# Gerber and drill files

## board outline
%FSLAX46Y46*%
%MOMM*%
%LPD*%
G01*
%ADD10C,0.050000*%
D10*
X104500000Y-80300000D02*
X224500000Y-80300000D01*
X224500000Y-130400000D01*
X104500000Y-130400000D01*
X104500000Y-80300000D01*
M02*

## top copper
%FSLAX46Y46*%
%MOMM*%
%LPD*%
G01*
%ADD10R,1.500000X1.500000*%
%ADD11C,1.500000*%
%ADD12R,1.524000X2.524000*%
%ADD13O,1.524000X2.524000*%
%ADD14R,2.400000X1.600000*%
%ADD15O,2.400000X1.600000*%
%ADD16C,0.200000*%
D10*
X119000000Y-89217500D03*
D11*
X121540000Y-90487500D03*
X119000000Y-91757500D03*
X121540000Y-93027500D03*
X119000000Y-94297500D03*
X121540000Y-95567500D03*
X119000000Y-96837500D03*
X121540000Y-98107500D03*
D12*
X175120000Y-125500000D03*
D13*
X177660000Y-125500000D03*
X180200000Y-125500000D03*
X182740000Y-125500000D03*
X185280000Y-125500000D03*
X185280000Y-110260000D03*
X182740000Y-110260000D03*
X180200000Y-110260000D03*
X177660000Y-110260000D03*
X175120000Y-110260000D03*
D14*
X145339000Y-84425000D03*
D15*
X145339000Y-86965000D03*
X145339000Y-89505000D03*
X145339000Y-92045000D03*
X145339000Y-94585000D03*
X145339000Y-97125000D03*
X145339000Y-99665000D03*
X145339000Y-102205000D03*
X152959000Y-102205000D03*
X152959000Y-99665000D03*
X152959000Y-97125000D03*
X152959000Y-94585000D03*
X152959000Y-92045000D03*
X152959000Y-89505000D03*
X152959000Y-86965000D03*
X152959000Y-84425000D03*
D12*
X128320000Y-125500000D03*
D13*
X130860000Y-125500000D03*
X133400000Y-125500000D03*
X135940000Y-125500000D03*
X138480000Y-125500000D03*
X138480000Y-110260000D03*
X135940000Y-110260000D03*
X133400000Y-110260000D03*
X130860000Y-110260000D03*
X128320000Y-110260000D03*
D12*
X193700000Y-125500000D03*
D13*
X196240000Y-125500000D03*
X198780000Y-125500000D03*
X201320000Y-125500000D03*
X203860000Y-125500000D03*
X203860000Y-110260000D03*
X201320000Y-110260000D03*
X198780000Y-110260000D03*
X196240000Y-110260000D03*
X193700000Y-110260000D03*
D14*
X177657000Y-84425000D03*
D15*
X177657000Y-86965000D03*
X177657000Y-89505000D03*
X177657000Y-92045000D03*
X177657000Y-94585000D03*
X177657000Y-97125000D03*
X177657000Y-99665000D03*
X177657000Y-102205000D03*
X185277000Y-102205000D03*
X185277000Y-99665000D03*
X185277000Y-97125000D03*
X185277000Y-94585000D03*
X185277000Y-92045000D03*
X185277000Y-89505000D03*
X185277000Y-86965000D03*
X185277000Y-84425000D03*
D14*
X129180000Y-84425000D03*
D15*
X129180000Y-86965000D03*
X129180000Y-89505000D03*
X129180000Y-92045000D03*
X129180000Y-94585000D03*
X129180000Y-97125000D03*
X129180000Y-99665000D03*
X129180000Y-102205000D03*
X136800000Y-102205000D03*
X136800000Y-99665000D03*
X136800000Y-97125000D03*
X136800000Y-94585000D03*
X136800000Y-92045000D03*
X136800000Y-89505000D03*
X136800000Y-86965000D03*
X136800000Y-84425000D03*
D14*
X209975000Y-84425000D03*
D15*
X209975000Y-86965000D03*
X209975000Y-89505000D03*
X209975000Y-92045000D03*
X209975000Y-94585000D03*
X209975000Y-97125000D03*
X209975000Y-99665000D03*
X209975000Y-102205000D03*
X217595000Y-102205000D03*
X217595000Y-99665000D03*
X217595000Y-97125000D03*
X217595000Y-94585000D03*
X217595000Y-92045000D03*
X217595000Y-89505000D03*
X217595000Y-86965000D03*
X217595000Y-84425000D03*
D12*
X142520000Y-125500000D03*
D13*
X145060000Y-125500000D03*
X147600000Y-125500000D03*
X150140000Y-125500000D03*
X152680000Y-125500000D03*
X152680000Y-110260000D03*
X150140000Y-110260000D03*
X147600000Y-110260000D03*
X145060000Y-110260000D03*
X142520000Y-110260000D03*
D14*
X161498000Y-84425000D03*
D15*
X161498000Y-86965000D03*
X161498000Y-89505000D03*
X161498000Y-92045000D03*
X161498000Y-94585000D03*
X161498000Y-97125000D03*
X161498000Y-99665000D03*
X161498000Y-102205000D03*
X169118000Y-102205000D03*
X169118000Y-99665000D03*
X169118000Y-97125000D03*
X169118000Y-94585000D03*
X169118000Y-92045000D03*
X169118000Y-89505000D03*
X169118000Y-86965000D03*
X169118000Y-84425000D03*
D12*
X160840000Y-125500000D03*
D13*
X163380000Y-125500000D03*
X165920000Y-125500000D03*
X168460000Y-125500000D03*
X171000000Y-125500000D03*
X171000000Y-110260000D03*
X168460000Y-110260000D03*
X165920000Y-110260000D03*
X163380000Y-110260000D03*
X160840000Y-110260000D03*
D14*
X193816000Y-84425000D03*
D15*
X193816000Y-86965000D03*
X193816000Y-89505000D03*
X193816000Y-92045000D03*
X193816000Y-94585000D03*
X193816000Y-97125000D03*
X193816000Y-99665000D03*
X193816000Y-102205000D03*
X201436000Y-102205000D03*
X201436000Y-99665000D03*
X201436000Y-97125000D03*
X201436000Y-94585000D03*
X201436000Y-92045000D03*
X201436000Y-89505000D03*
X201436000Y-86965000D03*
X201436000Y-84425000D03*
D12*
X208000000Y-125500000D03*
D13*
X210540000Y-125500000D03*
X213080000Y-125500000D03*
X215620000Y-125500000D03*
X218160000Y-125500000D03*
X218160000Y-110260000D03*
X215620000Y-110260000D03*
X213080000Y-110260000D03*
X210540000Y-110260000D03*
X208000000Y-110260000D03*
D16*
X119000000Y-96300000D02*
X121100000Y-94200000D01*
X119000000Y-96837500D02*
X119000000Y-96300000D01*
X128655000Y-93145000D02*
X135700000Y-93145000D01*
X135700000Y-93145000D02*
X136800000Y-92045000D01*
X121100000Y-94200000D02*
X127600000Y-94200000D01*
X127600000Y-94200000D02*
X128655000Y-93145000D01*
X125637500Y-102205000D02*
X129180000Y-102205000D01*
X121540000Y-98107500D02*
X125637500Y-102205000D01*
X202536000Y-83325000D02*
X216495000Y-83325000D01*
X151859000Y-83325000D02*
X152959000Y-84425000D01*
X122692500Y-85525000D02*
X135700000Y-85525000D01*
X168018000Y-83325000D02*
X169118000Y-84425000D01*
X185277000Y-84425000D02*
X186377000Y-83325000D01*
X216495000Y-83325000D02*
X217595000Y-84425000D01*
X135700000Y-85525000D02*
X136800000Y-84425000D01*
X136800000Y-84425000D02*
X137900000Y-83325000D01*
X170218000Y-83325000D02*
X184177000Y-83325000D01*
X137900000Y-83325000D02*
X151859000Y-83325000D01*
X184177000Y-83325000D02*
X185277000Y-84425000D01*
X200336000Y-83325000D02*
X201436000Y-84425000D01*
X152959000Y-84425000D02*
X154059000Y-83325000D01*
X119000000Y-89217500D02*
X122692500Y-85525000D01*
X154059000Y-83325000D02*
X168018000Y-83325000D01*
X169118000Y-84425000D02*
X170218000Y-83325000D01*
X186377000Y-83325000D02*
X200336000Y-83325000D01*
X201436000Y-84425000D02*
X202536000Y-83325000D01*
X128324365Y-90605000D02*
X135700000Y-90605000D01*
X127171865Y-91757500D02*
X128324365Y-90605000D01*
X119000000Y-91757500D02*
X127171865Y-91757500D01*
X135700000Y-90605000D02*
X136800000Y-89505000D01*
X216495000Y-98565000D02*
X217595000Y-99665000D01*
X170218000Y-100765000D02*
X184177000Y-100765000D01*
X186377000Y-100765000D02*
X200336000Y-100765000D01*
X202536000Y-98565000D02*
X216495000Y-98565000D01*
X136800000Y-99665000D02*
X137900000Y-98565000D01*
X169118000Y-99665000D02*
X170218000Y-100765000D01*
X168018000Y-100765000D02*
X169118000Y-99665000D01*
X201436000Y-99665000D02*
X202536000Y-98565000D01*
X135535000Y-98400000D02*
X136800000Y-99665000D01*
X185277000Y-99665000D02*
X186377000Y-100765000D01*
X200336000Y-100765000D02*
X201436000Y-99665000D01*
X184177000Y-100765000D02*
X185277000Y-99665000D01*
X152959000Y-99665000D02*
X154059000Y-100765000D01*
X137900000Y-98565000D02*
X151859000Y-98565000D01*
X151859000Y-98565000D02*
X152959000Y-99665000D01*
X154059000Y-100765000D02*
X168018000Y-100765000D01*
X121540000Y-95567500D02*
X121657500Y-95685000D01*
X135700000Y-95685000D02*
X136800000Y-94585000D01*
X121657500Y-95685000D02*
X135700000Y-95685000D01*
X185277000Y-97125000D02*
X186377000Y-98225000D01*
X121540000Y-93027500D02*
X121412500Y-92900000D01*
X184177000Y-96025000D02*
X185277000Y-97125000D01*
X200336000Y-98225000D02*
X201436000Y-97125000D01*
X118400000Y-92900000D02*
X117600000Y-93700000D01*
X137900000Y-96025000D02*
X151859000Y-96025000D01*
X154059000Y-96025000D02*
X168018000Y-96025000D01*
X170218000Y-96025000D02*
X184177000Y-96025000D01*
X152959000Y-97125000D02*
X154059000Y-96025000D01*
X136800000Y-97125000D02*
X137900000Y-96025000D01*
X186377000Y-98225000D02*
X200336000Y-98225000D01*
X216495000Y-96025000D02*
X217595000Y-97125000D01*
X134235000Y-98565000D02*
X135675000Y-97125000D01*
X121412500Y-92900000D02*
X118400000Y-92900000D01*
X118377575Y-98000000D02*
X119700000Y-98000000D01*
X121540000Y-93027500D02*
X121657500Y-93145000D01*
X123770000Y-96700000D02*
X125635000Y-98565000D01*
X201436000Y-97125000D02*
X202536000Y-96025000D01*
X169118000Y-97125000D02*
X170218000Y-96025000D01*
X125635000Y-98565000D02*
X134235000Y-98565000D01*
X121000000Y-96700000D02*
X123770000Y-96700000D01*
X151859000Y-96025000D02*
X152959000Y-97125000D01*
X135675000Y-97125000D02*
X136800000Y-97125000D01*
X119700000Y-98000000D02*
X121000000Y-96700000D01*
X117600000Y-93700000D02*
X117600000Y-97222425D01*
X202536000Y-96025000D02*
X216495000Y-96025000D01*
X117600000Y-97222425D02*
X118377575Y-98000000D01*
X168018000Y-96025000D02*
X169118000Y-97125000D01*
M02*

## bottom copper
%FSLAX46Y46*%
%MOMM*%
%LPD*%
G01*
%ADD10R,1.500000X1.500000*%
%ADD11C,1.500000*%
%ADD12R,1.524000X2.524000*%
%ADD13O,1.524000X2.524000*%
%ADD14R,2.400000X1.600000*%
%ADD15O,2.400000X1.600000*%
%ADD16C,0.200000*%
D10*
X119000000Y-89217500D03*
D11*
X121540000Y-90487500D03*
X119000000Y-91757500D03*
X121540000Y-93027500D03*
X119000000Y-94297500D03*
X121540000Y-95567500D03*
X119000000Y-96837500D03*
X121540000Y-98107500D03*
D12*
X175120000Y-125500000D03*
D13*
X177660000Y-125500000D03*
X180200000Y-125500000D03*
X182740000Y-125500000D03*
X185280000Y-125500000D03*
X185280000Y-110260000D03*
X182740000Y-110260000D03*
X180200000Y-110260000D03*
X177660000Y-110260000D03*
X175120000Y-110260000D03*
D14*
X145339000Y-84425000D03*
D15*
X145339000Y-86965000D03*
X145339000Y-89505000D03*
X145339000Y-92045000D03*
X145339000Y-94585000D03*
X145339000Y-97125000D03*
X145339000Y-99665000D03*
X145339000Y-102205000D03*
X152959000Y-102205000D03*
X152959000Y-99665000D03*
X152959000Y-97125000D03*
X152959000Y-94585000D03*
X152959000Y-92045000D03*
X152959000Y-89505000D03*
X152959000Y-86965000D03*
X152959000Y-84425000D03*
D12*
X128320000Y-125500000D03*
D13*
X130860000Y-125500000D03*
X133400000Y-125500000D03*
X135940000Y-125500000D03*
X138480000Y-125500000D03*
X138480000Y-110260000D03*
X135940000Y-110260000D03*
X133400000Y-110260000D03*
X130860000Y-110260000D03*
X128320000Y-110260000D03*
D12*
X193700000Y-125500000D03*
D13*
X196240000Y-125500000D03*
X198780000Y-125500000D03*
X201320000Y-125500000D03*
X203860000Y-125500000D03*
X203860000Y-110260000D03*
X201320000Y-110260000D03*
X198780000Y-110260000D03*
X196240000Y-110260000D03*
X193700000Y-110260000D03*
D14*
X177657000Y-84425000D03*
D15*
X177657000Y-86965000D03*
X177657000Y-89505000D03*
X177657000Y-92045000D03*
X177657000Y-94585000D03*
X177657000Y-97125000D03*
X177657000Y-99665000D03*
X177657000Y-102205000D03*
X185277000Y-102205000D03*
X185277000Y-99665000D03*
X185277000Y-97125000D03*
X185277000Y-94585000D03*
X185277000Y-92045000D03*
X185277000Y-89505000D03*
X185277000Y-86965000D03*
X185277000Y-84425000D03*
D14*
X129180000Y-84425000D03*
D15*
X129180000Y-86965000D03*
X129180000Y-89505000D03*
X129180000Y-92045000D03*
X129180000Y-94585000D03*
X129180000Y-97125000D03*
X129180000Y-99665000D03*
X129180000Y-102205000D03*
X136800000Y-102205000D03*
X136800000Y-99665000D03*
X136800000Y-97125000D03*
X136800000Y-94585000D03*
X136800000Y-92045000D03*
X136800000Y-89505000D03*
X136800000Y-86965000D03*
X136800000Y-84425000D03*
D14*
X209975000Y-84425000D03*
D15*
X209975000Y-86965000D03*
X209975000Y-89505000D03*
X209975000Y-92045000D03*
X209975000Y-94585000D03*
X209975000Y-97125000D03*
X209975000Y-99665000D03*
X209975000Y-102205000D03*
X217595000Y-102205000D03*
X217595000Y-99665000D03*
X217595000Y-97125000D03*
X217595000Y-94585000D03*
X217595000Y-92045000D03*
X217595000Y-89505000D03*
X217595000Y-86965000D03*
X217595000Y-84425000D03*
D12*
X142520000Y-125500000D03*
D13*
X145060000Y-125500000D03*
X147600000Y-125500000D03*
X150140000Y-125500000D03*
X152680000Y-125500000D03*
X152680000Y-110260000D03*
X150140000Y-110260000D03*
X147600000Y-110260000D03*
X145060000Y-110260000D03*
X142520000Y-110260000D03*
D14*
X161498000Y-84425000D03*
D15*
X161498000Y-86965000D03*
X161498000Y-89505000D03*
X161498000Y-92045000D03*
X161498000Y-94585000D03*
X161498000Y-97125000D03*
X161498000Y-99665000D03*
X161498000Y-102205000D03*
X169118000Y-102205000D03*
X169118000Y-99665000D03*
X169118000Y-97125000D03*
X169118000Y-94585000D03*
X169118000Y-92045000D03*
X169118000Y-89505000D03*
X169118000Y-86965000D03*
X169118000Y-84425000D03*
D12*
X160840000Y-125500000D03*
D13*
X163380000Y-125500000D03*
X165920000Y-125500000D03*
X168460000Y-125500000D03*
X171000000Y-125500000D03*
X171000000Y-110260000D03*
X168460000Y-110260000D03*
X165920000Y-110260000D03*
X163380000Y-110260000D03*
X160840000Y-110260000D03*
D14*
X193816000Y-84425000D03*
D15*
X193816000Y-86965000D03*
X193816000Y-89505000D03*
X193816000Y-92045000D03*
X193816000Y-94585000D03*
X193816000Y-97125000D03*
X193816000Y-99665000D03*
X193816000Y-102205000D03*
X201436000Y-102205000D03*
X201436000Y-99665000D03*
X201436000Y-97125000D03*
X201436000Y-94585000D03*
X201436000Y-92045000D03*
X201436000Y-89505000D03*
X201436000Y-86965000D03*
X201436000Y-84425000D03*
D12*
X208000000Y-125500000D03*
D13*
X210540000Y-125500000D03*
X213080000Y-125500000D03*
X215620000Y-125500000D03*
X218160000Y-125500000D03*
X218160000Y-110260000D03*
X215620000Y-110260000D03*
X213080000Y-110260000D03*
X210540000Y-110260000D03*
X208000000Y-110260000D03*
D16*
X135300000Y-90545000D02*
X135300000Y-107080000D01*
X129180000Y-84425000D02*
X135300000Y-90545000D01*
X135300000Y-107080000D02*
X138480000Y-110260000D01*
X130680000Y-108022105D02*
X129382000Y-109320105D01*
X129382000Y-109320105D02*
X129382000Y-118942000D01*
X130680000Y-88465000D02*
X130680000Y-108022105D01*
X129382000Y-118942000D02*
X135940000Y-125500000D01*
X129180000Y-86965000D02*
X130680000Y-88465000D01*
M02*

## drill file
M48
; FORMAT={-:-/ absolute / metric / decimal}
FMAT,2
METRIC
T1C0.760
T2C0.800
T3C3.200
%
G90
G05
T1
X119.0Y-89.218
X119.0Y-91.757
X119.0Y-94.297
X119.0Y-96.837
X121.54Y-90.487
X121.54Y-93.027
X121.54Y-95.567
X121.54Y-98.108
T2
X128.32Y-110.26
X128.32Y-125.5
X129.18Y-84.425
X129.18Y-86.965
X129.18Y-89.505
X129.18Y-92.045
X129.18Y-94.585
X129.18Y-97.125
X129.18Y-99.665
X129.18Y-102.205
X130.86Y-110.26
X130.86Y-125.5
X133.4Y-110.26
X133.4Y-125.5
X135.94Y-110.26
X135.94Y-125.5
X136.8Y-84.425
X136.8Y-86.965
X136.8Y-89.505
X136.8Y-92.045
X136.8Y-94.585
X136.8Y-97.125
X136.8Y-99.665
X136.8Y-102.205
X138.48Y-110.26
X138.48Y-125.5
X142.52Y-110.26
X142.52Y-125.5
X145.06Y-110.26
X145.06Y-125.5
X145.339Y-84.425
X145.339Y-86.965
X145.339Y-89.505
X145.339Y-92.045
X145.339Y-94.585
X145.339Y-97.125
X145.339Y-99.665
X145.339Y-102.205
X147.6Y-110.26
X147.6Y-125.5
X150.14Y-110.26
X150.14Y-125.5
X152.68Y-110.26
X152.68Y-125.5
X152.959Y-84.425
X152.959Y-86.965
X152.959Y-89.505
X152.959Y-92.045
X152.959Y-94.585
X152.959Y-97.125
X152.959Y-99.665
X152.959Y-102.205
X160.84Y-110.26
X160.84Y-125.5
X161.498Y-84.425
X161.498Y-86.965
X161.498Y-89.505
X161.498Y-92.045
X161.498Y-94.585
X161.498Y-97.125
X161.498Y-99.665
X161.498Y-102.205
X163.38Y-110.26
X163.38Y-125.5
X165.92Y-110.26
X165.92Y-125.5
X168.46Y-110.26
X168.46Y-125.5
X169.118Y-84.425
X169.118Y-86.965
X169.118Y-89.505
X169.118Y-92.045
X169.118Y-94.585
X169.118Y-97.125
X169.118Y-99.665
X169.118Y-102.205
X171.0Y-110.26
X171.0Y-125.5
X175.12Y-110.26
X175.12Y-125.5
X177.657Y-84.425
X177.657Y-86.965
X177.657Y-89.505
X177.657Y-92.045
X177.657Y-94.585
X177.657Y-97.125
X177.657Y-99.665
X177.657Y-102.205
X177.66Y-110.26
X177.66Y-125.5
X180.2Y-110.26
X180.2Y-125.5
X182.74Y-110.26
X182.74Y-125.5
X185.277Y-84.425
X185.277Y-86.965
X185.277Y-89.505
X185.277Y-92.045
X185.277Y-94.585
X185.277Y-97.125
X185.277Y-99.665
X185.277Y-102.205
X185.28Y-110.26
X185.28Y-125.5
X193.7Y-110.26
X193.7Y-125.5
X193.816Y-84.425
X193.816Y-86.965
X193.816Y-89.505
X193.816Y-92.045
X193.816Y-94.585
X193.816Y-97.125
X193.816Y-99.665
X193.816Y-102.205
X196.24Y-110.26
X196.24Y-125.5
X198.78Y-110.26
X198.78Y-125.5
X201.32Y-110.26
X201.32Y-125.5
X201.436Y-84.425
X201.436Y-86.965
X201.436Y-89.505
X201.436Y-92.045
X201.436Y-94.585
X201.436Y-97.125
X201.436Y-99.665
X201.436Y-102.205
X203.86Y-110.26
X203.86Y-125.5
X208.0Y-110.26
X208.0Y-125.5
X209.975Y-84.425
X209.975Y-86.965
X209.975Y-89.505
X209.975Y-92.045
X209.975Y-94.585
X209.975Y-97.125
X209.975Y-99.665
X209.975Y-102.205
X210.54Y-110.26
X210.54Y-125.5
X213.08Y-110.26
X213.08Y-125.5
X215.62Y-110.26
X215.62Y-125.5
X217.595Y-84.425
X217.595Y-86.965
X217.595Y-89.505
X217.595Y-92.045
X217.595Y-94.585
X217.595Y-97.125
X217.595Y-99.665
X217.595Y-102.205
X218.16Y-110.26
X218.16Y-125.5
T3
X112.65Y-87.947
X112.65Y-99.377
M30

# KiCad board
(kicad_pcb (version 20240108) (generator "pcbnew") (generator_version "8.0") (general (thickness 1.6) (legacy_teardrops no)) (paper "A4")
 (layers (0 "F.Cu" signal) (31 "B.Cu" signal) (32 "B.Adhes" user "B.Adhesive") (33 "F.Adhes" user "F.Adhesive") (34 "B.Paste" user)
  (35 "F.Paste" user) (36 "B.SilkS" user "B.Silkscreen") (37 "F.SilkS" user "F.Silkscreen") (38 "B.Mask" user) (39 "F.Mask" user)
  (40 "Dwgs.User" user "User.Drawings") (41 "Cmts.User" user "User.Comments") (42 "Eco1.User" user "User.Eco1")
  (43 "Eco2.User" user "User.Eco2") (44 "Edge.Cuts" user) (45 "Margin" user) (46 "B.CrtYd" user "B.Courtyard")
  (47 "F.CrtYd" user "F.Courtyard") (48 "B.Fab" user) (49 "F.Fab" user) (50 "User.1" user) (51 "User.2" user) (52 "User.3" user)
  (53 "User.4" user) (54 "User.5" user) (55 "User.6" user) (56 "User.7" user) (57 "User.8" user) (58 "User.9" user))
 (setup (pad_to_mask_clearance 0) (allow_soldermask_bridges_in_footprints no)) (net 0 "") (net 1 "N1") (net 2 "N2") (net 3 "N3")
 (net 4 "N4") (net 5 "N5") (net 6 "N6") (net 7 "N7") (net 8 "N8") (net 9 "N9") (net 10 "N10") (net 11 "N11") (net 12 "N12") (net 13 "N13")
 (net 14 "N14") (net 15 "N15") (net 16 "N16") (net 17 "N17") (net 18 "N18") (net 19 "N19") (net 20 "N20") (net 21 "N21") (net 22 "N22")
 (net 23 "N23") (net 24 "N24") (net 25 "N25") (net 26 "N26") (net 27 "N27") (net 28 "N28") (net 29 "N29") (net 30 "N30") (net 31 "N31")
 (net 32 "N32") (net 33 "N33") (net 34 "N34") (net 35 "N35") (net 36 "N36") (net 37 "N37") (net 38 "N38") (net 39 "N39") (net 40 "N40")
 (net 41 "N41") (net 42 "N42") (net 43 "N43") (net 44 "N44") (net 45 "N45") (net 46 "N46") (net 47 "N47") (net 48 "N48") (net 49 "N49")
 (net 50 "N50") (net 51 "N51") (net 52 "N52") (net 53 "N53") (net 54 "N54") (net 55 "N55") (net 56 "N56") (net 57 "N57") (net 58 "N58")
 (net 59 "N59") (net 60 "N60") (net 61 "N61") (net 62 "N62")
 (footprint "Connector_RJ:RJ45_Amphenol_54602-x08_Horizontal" (layer "F.Cu") (at 119 89.2175 -90)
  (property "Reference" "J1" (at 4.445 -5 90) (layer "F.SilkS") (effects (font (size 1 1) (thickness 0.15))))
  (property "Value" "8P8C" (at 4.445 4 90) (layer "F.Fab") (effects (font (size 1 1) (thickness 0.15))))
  (pad "" np_thru_hole circle (at -1.27 6.35 270) (size 3.2 3.2) (drill 3.2) (layers "*.Cu" "*.Mask"))
  (pad "" np_thru_hole circle (at 10.16 6.35 270) (size 3.2 3.2) (drill 3.2) (layers "*.Cu" "*.Mask"))
  (pad "1" thru_hole rect (at 0 0 270) (size 1.5 1.5) (drill 0.76) (layers "*.Cu" "*.Mask") (remove_unused_layers no) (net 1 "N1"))
  (pad "2" thru_hole circle (at 1.27 -2.54 270) (size 1.5 1.5) (drill 0.76) (layers "*.Cu" "*.Mask") (remove_unused_layers no) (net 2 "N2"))
  (pad "3" thru_hole circle (at 2.54 0 270) (size 1.5 1.5) (drill 0.76) (layers "*.Cu" "*.Mask") (remove_unused_layers no) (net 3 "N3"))
  (pad "4" thru_hole circle (at 3.81 -2.54 270) (size 1.5 1.5) (drill 0.76) (layers "*.Cu" "*.Mask") (remove_unused_layers no) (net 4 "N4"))
  (pad "5" thru_hole circle (at 5.08 0 270) (size 1.5 1.5) (drill 0.76) (layers "*.Cu" "*.Mask") (remove_unused_layers no) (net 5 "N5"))
  (pad "6" thru_hole circle (at 6.35 -2.54 270) (size 1.5 1.5) (drill 0.76) (layers "*.Cu" "*.Mask") (remove_unused_layers no) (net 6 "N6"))
  (pad "7" thru_hole circle (at 7.62 0 270) (size 1.5 1.5) (drill 0.76) (layers "*.Cu" "*.Mask") (remove_unused_layers no) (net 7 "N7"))
  (pad "8" thru_hole circle (at 8.89 -2.54 270) (size 1.5 1.5) (drill 0.76) (layers "*.Cu" "*.Mask") (remove_unused_layers no) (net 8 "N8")))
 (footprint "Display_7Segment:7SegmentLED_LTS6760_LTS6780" (layer "F.Cu") (at 175.12 125.5 90)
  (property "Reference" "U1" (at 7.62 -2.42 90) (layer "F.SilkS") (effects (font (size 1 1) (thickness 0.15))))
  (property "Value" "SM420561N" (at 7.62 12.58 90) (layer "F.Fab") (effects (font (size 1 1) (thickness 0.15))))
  (pad "1" thru_hole rect (at 0 0) (size 1.524 2.524) (drill 0.8) (layers "*.Cu" "*.Mask") (remove_unused_layers no) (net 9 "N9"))
  (pad "2" thru_hole oval (at 0 2.54) (size 1.524 2.524) (drill 0.8) (layers "*.Cu" "*.Mask") (remove_unused_layers no) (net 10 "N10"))
  (pad "3" thru_hole oval (at 0 5.08) (size 1.524 2.524) (drill 0.8) (layers "*.Cu" "*.Mask") (remove_unused_layers no) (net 8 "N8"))
  (pad "4" thru_hole oval (at 0 7.62) (size 1.524 2.524) (drill 0.8) (layers "*.Cu" "*.Mask") (remove_unused_layers no) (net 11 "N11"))
  (pad "5" thru_hole oval (at 0 10.16) (size 1.524 2.524) (drill 0.8) (layers "*.Cu" "*.Mask") (remove_unused_layers no) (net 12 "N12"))
  (pad "6" thru_hole oval (at 15.24 10.16) (size 1.524 2.524) (drill 0.8) (layers "*.Cu" "*.Mask") (remove_unused_layers no) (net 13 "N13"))
  (pad "7" thru_hole oval (at 15.24 7.62) (size 1.524 2.524) (drill 0.8) (layers "*.Cu" "*.Mask") (remove_unused_layers no) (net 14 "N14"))
  (pad "8" thru_hole oval (at 15.24 5.08) (size 1.524 2.524) (drill 0.8) (layers "*.Cu" "*.Mask") (remove_unused_layers no) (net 8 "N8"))
  (pad "9" thru_hole oval (at 15.24 2.54) (size 1.524 2.524) (drill 0.8) (layers "*.Cu" "*.Mask") (remove_unused_layers no) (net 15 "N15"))
  (pad "10" thru_hole oval (at 15.24 0) (size 1.524 2.524) (drill 0.8) (layers "*.Cu" "*.Mask") (remove_unused_layers no) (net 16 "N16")))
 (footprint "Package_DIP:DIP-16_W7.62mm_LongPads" (layer "F.Cu") (at 145.339 84.425)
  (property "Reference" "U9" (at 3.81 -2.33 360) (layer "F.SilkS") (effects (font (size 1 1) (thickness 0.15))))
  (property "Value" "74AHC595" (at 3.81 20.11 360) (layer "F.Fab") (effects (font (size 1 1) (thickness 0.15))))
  (pad "1" thru_hole rect (at 0 0) (size 2.4 1.6) (drill 0.8) (layers "*.Cu" "*.Mask") (remove_unused_layers no) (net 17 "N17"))
  (pad "2" thru_hole oval (at 0 2.54) (size 2.4 1.6) (drill 0.8) (layers "*.Cu" "*.Mask") (remove_unused_layers no) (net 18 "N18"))
  (pad "3" thru_hole oval (at 0 5.08) (size 2.4 1.6) (drill 0.8) (layers "*.Cu" "*.Mask") (remove_unused_layers no) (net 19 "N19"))
  (pad "4" thru_hole oval (at 0 7.62) (size 2.4 1.6) (drill 0.8) (layers "*.Cu" "*.Mask") (remove_unused_layers no) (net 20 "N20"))
  (pad "5" thru_hole oval (at 0 10.16) (size 2.4 1.6) (drill 0.8) (layers "*.Cu" "*.Mask") (remove_unused_layers no) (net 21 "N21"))
  (pad "6" thru_hole oval (at 0 12.7) (size 2.4 1.6) (drill 0.8) (layers "*.Cu" "*.Mask") (remove_unused_layers no) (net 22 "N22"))
  (pad "7" thru_hole oval (at 0 15.24) (size 2.4 1.6) (drill 0.8) (layers "*.Cu" "*.Mask") (remove_unused_layers no) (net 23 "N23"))
  (pad "8" thru_hole oval (at 0 17.78) (size 2.4 1.6) (drill 0.8) (layers "*.Cu" "*.Mask") (remove_unused_layers no) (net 8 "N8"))
  (pad "9" thru_hole oval (at 7.62 17.78) (size 2.4 1.6) (drill 0.8) (layers "*.Cu" "*.Mask") (remove_unused_layers no) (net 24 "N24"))
  (pad "10" thru_hole oval (at 7.62 15.24) (size 2.4 1.6) (drill 0.8) (layers "*.Cu" "*.Mask") (remove_unused_layers no) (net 5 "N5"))
  (pad "11" thru_hole oval (at 7.62 12.7) (size 2.4 1.6) (drill 0.8) (layers "*.Cu" "*.Mask") (remove_unused_layers no) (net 4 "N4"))
  (pad "12" thru_hole oval (at 7.62 10.16) (size 2.4 1.6) (drill 0.8) (layers "*.Cu" "*.Mask") (remove_unused_layers no) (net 6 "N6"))
  (pad "13" thru_hole oval (at 7.62 7.62) (size 2.4 1.6) (drill 0.8) (layers "*.Cu" "*.Mask") (remove_unused_layers no) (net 7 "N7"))
  (pad "14" thru_hole oval (at 7.62 5.08) (size 2.4 1.6) (drill 0.8) (layers "*.Cu" "*.Mask") (remove_unused_layers no) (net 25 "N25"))
  (pad "15" thru_hole oval (at 7.62 2.54) (size 2.4 1.6) (drill 0.8) (layers "*.Cu" "*.Mask") (remove_unused_layers no) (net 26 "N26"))
  (pad "16" thru_hole oval (at 7.62 0) (size 2.4 1.6) (drill 0.8) (layers "*.Cu" "*.Mask") (remove_unused_layers no) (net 1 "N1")))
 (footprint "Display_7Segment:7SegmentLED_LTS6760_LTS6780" (layer "F.Cu") (at 128.32 125.5 90)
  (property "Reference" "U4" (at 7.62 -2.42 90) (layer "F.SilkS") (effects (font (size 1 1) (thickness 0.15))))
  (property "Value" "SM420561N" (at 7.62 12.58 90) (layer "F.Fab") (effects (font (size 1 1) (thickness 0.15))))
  (pad "1" thru_hole rect (at 0 0) (size 1.524 2.524) (drill 0.8) (layers "*.Cu" "*.Mask") (remove_unused_layers no) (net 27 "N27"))
  (pad "2" thru_hole oval (at 0 2.54) (size 1.524 2.524) (drill 0.8) (layers "*.Cu" "*.Mask") (remove_unused_layers no) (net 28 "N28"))
  (pad "3" thru_hole oval (at 0 5.08) (size 1.524 2.524) (drill 0.8) (layers "*.Cu" "*.Mask") (remove_unused_layers no) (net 8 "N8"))
  (pad "4" thru_hole oval (at 0 7.62) (size 1.524 2.524) (drill 0.8) (layers "*.Cu" "*.Mask") (remove_unused_layers no) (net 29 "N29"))
  (pad "5" thru_hole oval (at 0 10.16) (size 1.524 2.524) (drill 0.8) (layers "*.Cu" "*.Mask") (remove_unused_layers no) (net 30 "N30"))
  (pad "6" thru_hole oval (at 15.24 10.16) (size 1.524 2.524) (drill 0.8) (layers "*.Cu" "*.Mask") (remove_unused_layers no) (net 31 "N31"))
  (pad "7" thru_hole oval (at 15.24 7.62) (size 1.524 2.524) (drill 0.8) (layers "*.Cu" "*.Mask") (remove_unused_layers no) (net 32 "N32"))
  (pad "8" thru_hole oval (at 15.24 5.08) (size 1.524 2.524) (drill 0.8) (layers "*.Cu" "*.Mask") (remove_unused_layers no) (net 8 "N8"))
  (pad "9" thru_hole oval (at 15.24 2.54) (size 1.524 2.524) (drill 0.8) (layers "*.Cu" "*.Mask") (remove_unused_layers no) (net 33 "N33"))
  (pad "10" thru_hole oval (at 15.24 0) (size 1.524 2.524) (drill 0.8) (layers "*.Cu" "*.Mask") (remove_unused_layers no) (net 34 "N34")))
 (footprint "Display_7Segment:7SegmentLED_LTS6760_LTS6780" (layer "F.Cu") (at 193.7 125.5 90)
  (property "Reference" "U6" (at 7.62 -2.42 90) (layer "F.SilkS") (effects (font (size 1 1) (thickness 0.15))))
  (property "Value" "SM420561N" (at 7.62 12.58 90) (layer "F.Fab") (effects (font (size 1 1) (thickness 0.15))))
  (pad "1" thru_hole rect (at 0 0) (size 1.524 2.524) (drill 0.8) (layers "*.Cu" "*.Mask") (remove_unused_layers no) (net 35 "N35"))
  (pad "2" thru_hole oval (at 0 2.54) (size 1.524 2.524) (drill 0.8) (layers "*.Cu" "*.Mask") (remove_unused_layers no) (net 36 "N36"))
  (pad "3" thru_hole oval (at 0 5.08) (size 1.524 2.524) (drill 0.8) (layers "*.Cu" "*.Mask") (remove_unused_layers no) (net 8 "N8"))
  (pad "4" thru_hole oval (at 0 7.62) (size 1.524 2.524) (drill 0.8) (layers "*.Cu" "*.Mask") (remove_unused_layers no) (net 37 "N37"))
  (pad "5" thru_hole oval (at 0 10.16) (size 1.524 2.524) (drill 0.8) (layers "*.Cu" "*.Mask") (remove_unused_layers no) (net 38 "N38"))
  (pad "6" thru_hole oval (at 15.24 10.16) (size 1.524 2.524) (drill 0.8) (layers "*.Cu" "*.Mask") (remove_unused_layers no) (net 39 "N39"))
  (pad "7" thru_hole oval (at 15.24 7.62) (size 1.524 2.524) (drill 0.8) (layers "*.Cu" "*.Mask") (remove_unused_layers no) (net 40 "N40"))
  (pad "8" thru_hole oval (at 15.24 5.08) (size 1.524 2.524) (drill 0.8) (layers "*.Cu" "*.Mask") (remove_unused_layers no) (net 8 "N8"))
  (pad "9" thru_hole oval (at 15.24 2.54) (size 1.524 2.524) (drill 0.8) (layers "*.Cu" "*.Mask") (remove_unused_layers no) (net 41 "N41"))
  (pad "10" thru_hole oval (at 15.24 0) (size 1.524 2.524) (drill 0.8) (layers "*.Cu" "*.Mask") (remove_unused_layers no) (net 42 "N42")))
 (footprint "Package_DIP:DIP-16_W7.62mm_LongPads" (layer "F.Cu") (at 177.657 84.425)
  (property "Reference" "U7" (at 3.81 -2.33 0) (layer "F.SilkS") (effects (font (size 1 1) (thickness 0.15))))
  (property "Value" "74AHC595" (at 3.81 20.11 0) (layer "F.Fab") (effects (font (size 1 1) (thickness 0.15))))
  (pad "1" thru_hole rect (at 0 0) (size 2.4 1.6) (drill 0.8) (layers "*.Cu" "*.Mask") (remove_unused_layers no) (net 13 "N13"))
  (pad "2" thru_hole oval (at 0 2.54) (size 2.4 1.6) (drill 0.8) (layers "*.Cu" "*.Mask") (remove_unused_layers no) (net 11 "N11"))
  (pad "3" thru_hole oval (at 0 5.08) (size 2.4 1.6) (drill 0.8) (layers "*.Cu" "*.Mask") (remove_unused_layers no) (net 10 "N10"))
  (pad "4" thru_hole oval (at 0 7.62) (size 2.4 1.6) (drill 0.8) (layers "*.Cu" "*.Mask") (remove_unused_layers no) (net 9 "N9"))
  (pad "5" thru_hole oval (at 0 10.16) (size 2.4 1.6) (drill 0.8) (layers "*.Cu" "*.Mask") (remove_unused_layers no) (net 15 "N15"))
  (pad "6" thru_hole oval (at 0 12.7) (size 2.4 1.6) (drill 0.8) (layers "*.Cu" "*.Mask") (remove_unused_layers no) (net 16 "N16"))
  (pad "7" thru_hole oval (at 0 15.24) (size 2.4 1.6) (drill 0.8) (layers "*.Cu" "*.Mask") (remove_unused_layers no) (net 12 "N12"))
  (pad "8" thru_hole oval (at 0 17.78) (size 2.4 1.6) (drill 0.8) (layers "*.Cu" "*.Mask") (remove_unused_layers no) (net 8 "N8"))
  (pad "9" thru_hole oval (at 7.62 17.78) (size 2.4 1.6) (drill 0.8) (layers "*.Cu" "*.Mask") (remove_unused_layers no) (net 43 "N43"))
  (pad "10" thru_hole oval (at 7.62 15.24) (size 2.4 1.6) (drill 0.8) (layers "*.Cu" "*.Mask") (remove_unused_layers no) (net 5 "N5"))
  (pad "11" thru_hole oval (at 7.62 12.7) (size 2.4 1.6) (drill 0.8) (layers "*.Cu" "*.Mask") (remove_unused_layers no) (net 4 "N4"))
  (pad "12" thru_hole oval (at 7.62 10.16) (size 2.4 1.6) (drill 0.8) (layers "*.Cu" "*.Mask") (remove_unused_layers no) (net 6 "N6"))
  (pad "13" thru_hole oval (at 7.62 7.62) (size 2.4 1.6) (drill 0.8) (layers "*.Cu" "*.Mask") (remove_unused_layers no) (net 7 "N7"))
  (pad "14" thru_hole oval (at 7.62 5.08) (size 2.4 1.6) (drill 0.8) (layers "*.Cu" "*.Mask") (remove_unused_layers no) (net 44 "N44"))
  (pad "15" thru_hole oval (at 7.62 2.54) (size 2.4 1.6) (drill 0.8) (layers "*.Cu" "*.Mask") (remove_unused_layers no) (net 14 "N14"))
  (pad "16" thru_hole oval (at 7.62 0) (size 2.4 1.6) (drill 0.8) (layers "*.Cu" "*.Mask") (remove_unused_layers no) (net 1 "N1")))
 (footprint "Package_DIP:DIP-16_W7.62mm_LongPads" (layer "F.Cu") (at 129.18 84.425)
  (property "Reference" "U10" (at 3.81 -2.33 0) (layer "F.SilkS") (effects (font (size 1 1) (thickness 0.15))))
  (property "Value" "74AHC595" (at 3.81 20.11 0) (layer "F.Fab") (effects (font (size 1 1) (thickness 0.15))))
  (pad "1" thru_hole rect (at 0 0) (size 2.4 1.6) (drill 0.8) (layers "*.Cu" "*.Mask") (remove_unused_layers no) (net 31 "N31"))
  (pad "2" thru_hole oval (at 0 2.54) (size 2.4 1.6) (drill 0.8) (layers "*.Cu" "*.Mask") (remove_unused_layers no) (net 29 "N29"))
  (pad "3" thru_hole oval (at 0 5.08) (size 2.4 1.6) (drill 0.8) (layers "*.Cu" "*.Mask") (remove_unused_layers no) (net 28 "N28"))
  (pad "4" thru_hole oval (at 0 7.62) (size 2.4 1.6) (drill 0.8) (layers "*.Cu" "*.Mask") (remove_unused_layers no) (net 27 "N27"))
  (pad "5" thru_hole oval (at 0 10.16) (size 2.4 1.6) (drill 0.8) (layers "*.Cu" "*.Mask") (remove_unused_layers no) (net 33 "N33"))
  (pad "6" thru_hole oval (at 0 12.7) (size 2.4 1.6) (drill 0.8) (layers "*.Cu" "*.Mask") (remove_unused_layers no) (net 34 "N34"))
  (pad "7" thru_hole oval (at 0 15.24) (size 2.4 1.6) (drill 0.8) (layers "*.Cu" "*.Mask") (remove_unused_layers no) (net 30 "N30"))
  (pad "8" thru_hole oval (at 0 17.78) (size 2.4 1.6) (drill 0.8) (layers "*.Cu" "*.Mask") (remove_unused_layers no) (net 8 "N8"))
  (pad "9" thru_hole oval (at 7.62 17.78) (size 2.4 1.6) (drill 0.8) (layers "*.Cu" "*.Mask") (remove_unused_layers no) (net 25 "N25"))
  (pad "10" thru_hole oval (at 7.62 15.24) (size 2.4 1.6) (drill 0.8) (layers "*.Cu" "*.Mask") (remove_unused_layers no) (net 5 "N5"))
  (pad "11" thru_hole oval (at 7.62 12.7) (size 2.4 1.6) (drill 0.8) (layers "*.Cu" "*.Mask") (remove_unused_layers no) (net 4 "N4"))
  (pad "12" thru_hole oval (at 7.62 10.16) (size 2.4 1.6) (drill 0.8) (layers "*.Cu" "*.Mask") (remove_unused_layers no) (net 6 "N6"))
  (pad "13" thru_hole oval (at 7.62 7.62) (size 2.4 1.6) (drill 0.8) (layers "*.Cu" "*.Mask") (remove_unused_layers no) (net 7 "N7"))
  (pad "14" thru_hole oval (at 7.62 5.08) (size 2.4 1.6) (drill 0.8) (layers "*.Cu" "*.Mask") (remove_unused_layers no) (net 3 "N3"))
  (pad "15" thru_hole oval (at 7.62 2.54) (size 2.4 1.6) (drill 0.8) (layers "*.Cu" "*.Mask") (remove_unused_layers no) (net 32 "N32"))
  (pad "16" thru_hole oval (at 7.62 0) (size 2.4 1.6) (drill 0.8) (layers "*.Cu" "*.Mask") (remove_unused_layers no) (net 1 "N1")))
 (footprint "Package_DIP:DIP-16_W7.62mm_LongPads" (layer "F.Cu") (at 209.975 84.425)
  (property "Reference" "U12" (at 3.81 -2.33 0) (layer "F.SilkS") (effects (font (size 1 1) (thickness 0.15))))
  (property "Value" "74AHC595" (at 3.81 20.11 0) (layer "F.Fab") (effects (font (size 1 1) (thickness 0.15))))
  (pad "1" thru_hole rect (at 0 0) (size 2.4 1.6) (drill 0.8) (layers "*.Cu" "*.Mask") (remove_unused_layers no) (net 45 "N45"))
  (pad "2" thru_hole oval (at 0 2.54) (size 2.4 1.6) (drill 0.8) (layers "*.Cu" "*.Mask") (remove_unused_layers no) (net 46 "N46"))
  (pad "3" thru_hole oval (at 0 5.08) (size 2.4 1.6) (drill 0.8) (layers "*.Cu" "*.Mask") (remove_unused_layers no) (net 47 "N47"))
  (pad "4" thru_hole oval (at 0 7.62) (size 2.4 1.6) (drill 0.8) (layers "*.Cu" "*.Mask") (remove_unused_layers no) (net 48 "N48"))
  (pad "5" thru_hole oval (at 0 10.16) (size 2.4 1.6) (drill 0.8) (layers "*.Cu" "*.Mask") (remove_unused_layers no) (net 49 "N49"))
  (pad "6" thru_hole oval (at 0 12.7) (size 2.4 1.6) (drill 0.8) (layers "*.Cu" "*.Mask") (remove_unused_layers no) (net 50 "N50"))
  (pad "7" thru_hole oval (at 0 15.24) (size 2.4 1.6) (drill 0.8) (layers "*.Cu" "*.Mask") (remove_unused_layers no) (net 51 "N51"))
  (pad "8" thru_hole oval (at 0 17.78) (size 2.4 1.6) (drill 0.8) (layers "*.Cu" "*.Mask") (remove_unused_layers no) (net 8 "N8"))
  (pad "9" thru_hole oval (at 7.62 17.78) (size 2.4 1.6) (drill 0.8) (layers "*.Cu" "*.Mask") (remove_unused_layers no) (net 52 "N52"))
  (pad "10" thru_hole oval (at 7.62 15.24) (size 2.4 1.6) (drill 0.8) (layers "*.Cu" "*.Mask") (remove_unused_layers no) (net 5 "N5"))
  (pad "11" thru_hole oval (at 7.62 12.7) (size 2.4 1.6) (drill 0.8) (layers "*.Cu" "*.Mask") (remove_unused_layers no) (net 4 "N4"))
  (pad "12" thru_hole oval (at 7.62 10.16) (size 2.4 1.6) (drill 0.8) (layers "*.Cu" "*.Mask") (remove_unused_layers no) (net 6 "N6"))
  (pad "13" thru_hole oval (at 7.62 7.62) (size 2.4 1.6) (drill 0.8) (layers "*.Cu" "*.Mask") (remove_unused_layers no) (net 7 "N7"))
  (pad "14" thru_hole oval (at 7.62 5.08) (size 2.4 1.6) (drill 0.8) (layers "*.Cu" "*.Mask") (remove_unused_layers no) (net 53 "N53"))
  (pad "15" thru_hole oval (at 7.62 2.54) (size 2.4 1.6) (drill 0.8) (layers "*.Cu" "*.Mask") (remove_unused_layers no) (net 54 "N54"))
  (pad "16" thru_hole oval (at 7.62 0) (size 2.4 1.6) (drill 0.8) (layers "*.Cu" "*.Mask") (remove_unused_layers no) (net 1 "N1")))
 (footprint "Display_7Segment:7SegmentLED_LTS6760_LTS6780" (layer "F.Cu") (at 142.52 125.5 90)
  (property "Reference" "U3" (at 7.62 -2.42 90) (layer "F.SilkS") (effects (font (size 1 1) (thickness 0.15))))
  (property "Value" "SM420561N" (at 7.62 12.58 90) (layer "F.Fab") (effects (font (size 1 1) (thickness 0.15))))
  (pad "1" thru_hole rect (at 0 0) (size 1.524 2.524) (drill 0.8) (layers "*.Cu" "*.Mask") (remove_unused_layers no) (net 20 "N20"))
  (pad "2" thru_hole oval (at 0 2.54) (size 1.524 2.524) (drill 0.8) (layers "*.Cu" "*.Mask") (remove_unused_layers no) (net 19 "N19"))
  (pad "3" thru_hole oval (at 0 5.08) (size 1.524 2.524) (drill 0.8) (layers "*.Cu" "*.Mask") (remove_unused_layers no) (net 8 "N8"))
  (pad "4" thru_hole oval (at 0 7.62) (size 1.524 2.524) (drill 0.8) (layers "*.Cu" "*.Mask") (remove_unused_layers no) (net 18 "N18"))
  (pad "5" thru_hole oval (at 0 10.16) (size 1.524 2.524) (drill 0.8) (layers "*.Cu" "*.Mask") (remove_unused_layers no) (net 23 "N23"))
  (pad "6" thru_hole oval (at 15.24 10.16) (size 1.524 2.524) (drill 0.8) (layers "*.Cu" "*.Mask") (remove_unused_layers no) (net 17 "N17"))
  (pad "7" thru_hole oval (at 15.24 7.62) (size 1.524 2.524) (drill 0.8) (layers "*.Cu" "*.Mask") (remove_unused_layers no) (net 26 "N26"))
  (pad "8" thru_hole oval (at 15.24 5.08) (size 1.524 2.524) (drill 0.8) (layers "*.Cu" "*.Mask") (remove_unused_layers no) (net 8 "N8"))
  (pad "9" thru_hole oval (at 15.24 2.54) (size 1.524 2.524) (drill 0.8) (layers "*.Cu" "*.Mask") (remove_unused_layers no) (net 21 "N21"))
  (pad "10" thru_hole oval (at 15.24 0) (size 1.524 2.524) (drill 0.8) (layers "*.Cu" "*.Mask") (remove_unused_layers no) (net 22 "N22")))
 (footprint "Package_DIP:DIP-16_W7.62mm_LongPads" (layer "F.Cu") (at 161.498 84.425)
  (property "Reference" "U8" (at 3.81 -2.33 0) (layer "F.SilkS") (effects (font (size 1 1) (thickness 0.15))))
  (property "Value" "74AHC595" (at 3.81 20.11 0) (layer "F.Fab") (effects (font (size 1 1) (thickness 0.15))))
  (pad "1" thru_hole rect (at 0 0) (size 2.4 1.6) (drill 0.8) (layers "*.Cu" "*.Mask") (remove_unused_layers no) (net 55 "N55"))
  (pad "2" thru_hole oval (at 0 2.54) (size 2.4 1.6) (drill 0.8) (layers "*.Cu" "*.Mask") (remove_unused_layers no) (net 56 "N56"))
  (pad "3" thru_hole oval (at 0 5.08) (size 2.4 1.6) (drill 0.8) (layers "*.Cu" "*.Mask") (remove_unused_layers no) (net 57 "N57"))
  (pad "4" thru_hole oval (at 0 7.62) (size 2.4 1.6) (drill 0.8) (layers "*.Cu" "*.Mask") (remove_unused_layers no) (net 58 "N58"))
  (pad "5" thru_hole oval (at 0 10.16) (size 2.4 1.6) (drill 0.8) (layers "*.Cu" "*.Mask") (remove_unused_layers no) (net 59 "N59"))
  (pad "6" thru_hole oval (at 0 12.7) (size 2.4 1.6) (drill 0.8) (layers "*.Cu" "*.Mask") (remove_unused_layers no) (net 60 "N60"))
  (pad "7" thru_hole oval (at 0 15.24) (size 2.4 1.6) (drill 0.8) (layers "*.Cu" "*.Mask") (remove_unused_layers no) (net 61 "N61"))
  (pad "8" thru_hole oval (at 0 17.78) (size 2.4 1.6) (drill 0.8) (layers "*.Cu" "*.Mask") (remove_unused_layers no) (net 8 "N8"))
  (pad "9" thru_hole oval (at 7.62 17.78) (size 2.4 1.6) (drill 0.8) (layers "*.Cu" "*.Mask") (remove_unused_layers no) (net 44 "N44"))
  (pad "10" thru_hole oval (at 7.62 15.24) (size 2.4 1.6) (drill 0.8) (layers "*.Cu" "*.Mask") (remove_unused_layers no) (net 5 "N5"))
  (pad "11" thru_hole oval (at 7.62 12.7) (size 2.4 1.6) (drill 0.8) (layers "*.Cu" "*.Mask") (remove_unused_layers no) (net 4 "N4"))
  (pad "12" thru_hole oval (at 7.62 10.16) (size 2.4 1.6) (drill 0.8) (layers "*.Cu" "*.Mask") (remove_unused_layers no) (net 6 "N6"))
  (pad "13" thru_hole oval (at 7.62 7.62) (size 2.4 1.6) (drill 0.8) (layers "*.Cu" "*.Mask") (remove_unused_layers no) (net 7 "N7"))
  (pad "14" thru_hole oval (at 7.62 5.08) (size 2.4 1.6) (drill 0.8) (layers "*.Cu" "*.Mask") (remove_unused_layers no) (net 24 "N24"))
  (pad "15" thru_hole oval (at 7.62 2.54) (size 2.4 1.6) (drill 0.8) (layers "*.Cu" "*.Mask") (remove_unused_layers no) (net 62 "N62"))
  (pad "16" thru_hole oval (at 7.62 0) (size 2.4 1.6) (drill 0.8) (layers "*.Cu" "*.Mask") (remove_unused_layers no) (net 1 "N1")))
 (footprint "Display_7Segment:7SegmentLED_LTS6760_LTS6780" (layer "F.Cu") (at 160.84 125.5 90)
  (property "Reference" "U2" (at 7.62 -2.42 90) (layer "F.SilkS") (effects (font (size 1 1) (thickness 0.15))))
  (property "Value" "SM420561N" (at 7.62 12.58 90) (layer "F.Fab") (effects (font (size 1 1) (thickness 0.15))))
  (pad "1" thru_hole rect (at 0 0) (size 1.524 2.524) (drill 0.8) (layers "*.Cu" "*.Mask") (remove_unused_layers no) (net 58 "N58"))
  (pad "2" thru_hole oval (at 0 2.54) (size 1.524 2.524) (drill 0.8) (layers "*.Cu" "*.Mask") (remove_unused_layers no) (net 57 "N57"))
  (pad "3" thru_hole oval (at 0 5.08) (size 1.524 2.524) (drill 0.8) (layers "*.Cu" "*.Mask") (remove_unused_layers no) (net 8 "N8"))
  (pad "4" thru_hole oval (at 0 7.62) (size 1.524 2.524) (drill 0.8) (layers "*.Cu" "*.Mask") (remove_unused_layers no) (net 56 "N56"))
  (pad "5" thru_hole oval (at 0 10.16) (size 1.524 2.524) (drill 0.8) (layers "*.Cu" "*.Mask") (remove_unused_layers no) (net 61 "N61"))
  (pad "6" thru_hole oval (at 15.24 10.16) (size 1.524 2.524) (drill 0.8) (layers "*.Cu" "*.Mask") (remove_unused_layers no) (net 55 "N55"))
  (pad "7" thru_hole oval (at 15.24 7.62) (size 1.524 2.524) (drill 0.8) (layers "*.Cu" "*.Mask") (remove_unused_layers no) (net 62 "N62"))
  (pad "8" thru_hole oval (at 15.24 5.08) (size 1.524 2.524) (drill 0.8) (layers "*.Cu" "*.Mask") (remove_unused_layers no) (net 8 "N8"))
  (pad "9" thru_hole oval (at 15.24 2.54) (size 1.524 2.524) (drill 0.8) (layers "*.Cu" "*.Mask") (remove_unused_layers no) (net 59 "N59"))
  (pad "10" thru_hole oval (at 15.24 0) (size 1.524 2.524) (drill 0.8) (layers "*.Cu" "*.Mask") (remove_unused_layers no) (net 60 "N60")))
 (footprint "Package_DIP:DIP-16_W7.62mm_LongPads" (layer "F.Cu") (at 193.816 84.425)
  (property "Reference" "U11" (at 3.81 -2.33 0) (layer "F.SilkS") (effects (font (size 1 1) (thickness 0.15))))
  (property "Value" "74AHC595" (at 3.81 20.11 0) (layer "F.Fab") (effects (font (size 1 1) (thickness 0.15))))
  (pad "1" thru_hole rect (at 0 0) (size 2.4 1.6) (drill 0.8) (layers "*.Cu" "*.Mask") (remove_unused_layers no) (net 39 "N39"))
  (pad "2" thru_hole oval (at 0 2.54) (size 2.4 1.6) (drill 0.8) (layers "*.Cu" "*.Mask") (remove_unused_layers no) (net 37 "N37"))
  (pad "3" thru_hole oval (at 0 5.08) (size 2.4 1.6) (drill 0.8) (layers "*.Cu" "*.Mask") (remove_unused_layers no) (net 36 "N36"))
  (pad "4" thru_hole oval (at 0 7.62) (size 2.4 1.6) (drill 0.8) (layers "*.Cu" "*.Mask") (remove_unused_layers no) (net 35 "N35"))
  (pad "5" thru_hole oval (at 0 10.16) (size 2.4 1.6) (drill 0.8) (layers "*.Cu" "*.Mask") (remove_unused_layers no) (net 41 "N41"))
  (pad "6" thru_hole oval (at 0 12.7) (size 2.4 1.6) (drill 0.8) (layers "*.Cu" "*.Mask") (remove_unused_layers no) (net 42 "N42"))
  (pad "7" thru_hole oval (at 0 15.24) (size 2.4 1.6) (drill 0.8) (layers "*.Cu" "*.Mask") (remove_unused_layers no) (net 38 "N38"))
  (pad "8" thru_hole oval (at 0 17.78) (size 2.4 1.6) (drill 0.8) (layers "*.Cu" "*.Mask") (remove_unused_layers no) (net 8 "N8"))
  (pad "9" thru_hole oval (at 7.62 17.78) (size 2.4 1.6) (drill 0.8) (layers "*.Cu" "*.Mask") (remove_unused_layers no) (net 53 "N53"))
  (pad "10" thru_hole oval (at 7.62 15.24) (size 2.4 1.6) (drill 0.8) (layers "*.Cu" "*.Mask") (remove_unused_layers no) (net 5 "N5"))
  (pad "11" thru_hole oval (at 7.62 12.7) (size 2.4 1.6) (drill 0.8) (layers "*.Cu" "*.Mask") (remove_unused_layers no) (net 4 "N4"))
  (pad "12" thru_hole oval (at 7.62 10.16) (size 2.4 1.6) (drill 0.8) (layers "*.Cu" "*.Mask") (remove_unused_layers no) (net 6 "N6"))
  (pad "13" thru_hole oval (at 7.62 7.62) (size 2.4 1.6) (drill 0.8) (layers "*.Cu" "*.Mask") (remove_unused_layers no) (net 7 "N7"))
  (pad "14" thru_hole oval (at 7.62 5.08) (size 2.4 1.6) (drill 0.8) (layers "*.Cu" "*.Mask") (remove_unused_layers no) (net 43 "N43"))
  (pad "15" thru_hole oval (at 7.62 2.54) (size 2.4 1.6) (drill 0.8) (layers "*.Cu" "*.Mask") (remove_unused_layers no) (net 40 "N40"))
  (pad "16" thru_hole oval (at 7.62 0) (size 2.4 1.6) (drill 0.8) (layers "*.Cu" "*.Mask") (remove_unused_layers no) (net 1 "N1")))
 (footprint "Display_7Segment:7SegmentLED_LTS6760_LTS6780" (layer "F.Cu") (at 208 125.5 90)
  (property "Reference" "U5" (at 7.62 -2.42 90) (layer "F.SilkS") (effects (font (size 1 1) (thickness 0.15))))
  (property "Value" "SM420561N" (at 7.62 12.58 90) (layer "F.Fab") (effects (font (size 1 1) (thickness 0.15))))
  (pad "1" thru_hole rect (at 0 0) (size 1.524 2.524) (drill 0.8) (layers "*.Cu" "*.Mask") (remove_unused_layers no) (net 48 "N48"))
  (pad "2" thru_hole oval (at 0 2.54) (size 1.524 2.524) (drill 0.8) (layers "*.Cu" "*.Mask") (remove_unused_layers no) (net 47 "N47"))
  (pad "3" thru_hole oval (at 0 5.08) (size 1.524 2.524) (drill 0.8) (layers "*.Cu" "*.Mask") (remove_unused_layers no) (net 8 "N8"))
  (pad "4" thru_hole oval (at 0 7.62) (size 1.524 2.524) (drill 0.8) (layers "*.Cu" "*.Mask") (remove_unused_layers no) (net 46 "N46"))
  (pad "5" thru_hole oval (at 0 10.16) (size 1.524 2.524) (drill 0.8) (layers "*.Cu" "*.Mask") (remove_unused_layers no) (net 51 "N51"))
  (pad "6" thru_hole oval (at 15.24 10.16) (size 1.524 2.524) (drill 0.8) (layers "*.Cu" "*.Mask") (remove_unused_layers no) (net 45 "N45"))
  (pad "7" thru_hole oval (at 15.24 7.62) (size 1.524 2.524) (drill 0.8) (layers "*.Cu" "*.Mask") (remove_unused_layers no) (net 54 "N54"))
  (pad "8" thru_hole oval (at 15.24 5.08) (size 1.524 2.524) (drill 0.8) (layers "*.Cu" "*.Mask") (remove_unused_layers no) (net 8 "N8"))
  (pad "9" thru_hole oval (at 15.24 2.54) (size 1.524 2.524) (drill 0.8) (layers "*.Cu" "*.Mask") (remove_unused_layers no) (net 49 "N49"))
  (pad "10" thru_hole oval (at 15.24 0) (size 1.524 2.524) (drill 0.8) (layers "*.Cu" "*.Mask") (remove_unused_layers no) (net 50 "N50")))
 (gr_rect (start 104.5 80.3) (end 224.5 130.4) (stroke (width 0.05) (type default)) (fill none) (layer "Edge.Cuts"))
 (segment (start 119 96.3) (end 121.1 94.2) (width 0.2) (layer "F.Cu") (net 7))
 (segment (start 119 96.8375) (end 119 96.3) (width 0.2) (layer "F.Cu") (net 7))
 (segment (start 128.655 93.145) (end 135.7 93.145) (width 0.2) (layer "F.Cu") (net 7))
 (segment (start 135.7 93.145) (end 136.8 92.045) (width 0.2) (layer "F.Cu") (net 7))
 (segment (start 121.1 94.2) (end 127.6 94.2) (width 0.2) (layer "F.Cu") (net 7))
 (segment (start 127.6 94.2) (end 128.655 93.145) (width 0.2) (layer "F.Cu") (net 7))
 (segment (start 125.6375 102.205) (end 129.18 102.205) (width 0.2) (layer "F.Cu") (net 8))
 (segment (start 121.54 98.1075) (end 125.6375 102.205) (width 0.2) (layer "F.Cu") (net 8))
 (segment (start 202.536 83.325) (end 216.495 83.325) (width 0.2) (layer "F.Cu") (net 1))
 (segment (start 151.859 83.325) (end 152.959 84.425) (width 0.2) (layer "F.Cu") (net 1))
 (segment (start 122.6925 85.525) (end 135.7 85.525) (width 0.2) (layer "F.Cu") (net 1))
 (segment (start 168.018 83.325) (end 169.118 84.425) (width 0.2) (layer "F.Cu") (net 1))
 (segment (start 185.277 84.425) (end 186.377 83.325) (width 0.2) (layer "F.Cu") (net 1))
 (segment (start 216.495 83.325) (end 217.595 84.425) (width 0.2) (layer "F.Cu") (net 1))
 (segment (start 135.7 85.525) (end 136.8 84.425) (width 0.2) (layer "F.Cu") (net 1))
 (segment (start 136.8 84.425) (end 137.9 83.325) (width 0.2) (layer "F.Cu") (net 1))
 (segment (start 170.218 83.325) (end 184.177 83.325) (width 0.2) (layer "F.Cu") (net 1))
 (segment (start 137.9 83.325) (end 151.859 83.325) (width 0.2) (layer "F.Cu") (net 1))
 (segment (start 184.177 83.325) (end 185.277 84.425) (width 0.2) (layer "F.Cu") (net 1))
 (segment (start 200.336 83.325) (end 201.436 84.425) (width 0.2) (layer "F.Cu") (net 1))
 (segment (start 152.959 84.425) (end 154.059 83.325) (width 0.2) (layer "F.Cu") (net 1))
 (segment (start 119 89.2175) (end 122.6925 85.525) (width 0.2) (layer "F.Cu") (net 1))
 (segment (start 154.059 83.325) (end 168.018 83.325) (width 0.2) (layer "F.Cu") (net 1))
 (segment (start 169.118 84.425) (end 170.218 83.325) (width 0.2) (layer "F.Cu") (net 1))
 (segment (start 186.377 83.325) (end 200.336 83.325) (width 0.2) (layer "F.Cu") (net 1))
 (segment (start 201.436 84.425) (end 202.536 83.325) (width 0.2) (layer "F.Cu") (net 1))
 (segment (start 128.324365 90.605) (end 135.7 90.605) (width 0.2) (layer "F.Cu") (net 3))
 (segment (start 127.171865 91.7575) (end 128.324365 90.605) (width 0.2) (layer "F.Cu") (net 3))
 (segment (start 119 91.7575) (end 127.171865 91.7575) (width 0.2) (layer "F.Cu") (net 3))
 (segment (start 135.7 90.605) (end 136.8 89.505) (width 0.2) (layer "F.Cu") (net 3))
 (segment (start 216.495 98.565) (end 217.595 99.665) (width 0.2) (layer "F.Cu") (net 5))
 (segment (start 170.218 100.765) (end 184.177 100.765) (width 0.2) (layer "F.Cu") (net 5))
 (segment (start 186.377 100.765) (end 200.336 100.765) (width 0.2) (layer "F.Cu") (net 5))
 (segment (start 202.536 98.565) (end 216.495 98.565) (width 0.2) (layer "F.Cu") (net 5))
 (segment (start 136.8 99.665) (end 137.9 98.565) (width 0.2) (layer "F.Cu") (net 5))
 (segment (start 169.118 99.665) (end 170.218 100.765) (width 0.2) (layer "F.Cu") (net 5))
 (segment (start 168.018 100.765) (end 169.118 99.665) (width 0.2) (layer "F.Cu") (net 5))
 (segment (start 201.436 99.665) (end 202.536 98.565) (width 0.2) (layer "F.Cu") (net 5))
 (segment (start 135.535 98.4) (end 136.8 99.665) (width 0.2) (layer "F.Cu") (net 5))
 (segment (start 185.277 99.665) (end 186.377 100.765) (width 0.2) (layer "F.Cu") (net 5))
 (segment (start 200.336 100.765) (end 201.436 99.665) (width 0.2) (layer "F.Cu") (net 5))
 (segment (start 184.177 100.765) (end 185.277 99.665) (width 0.2) (layer "F.Cu") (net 5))
 (segment (start 152.959 99.665) (end 154.059 100.765) (width 0.2) (layer "F.Cu") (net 5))
 (segment (start 137.9 98.565) (end 151.859 98.565) (width 0.2) (layer "F.Cu") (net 5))
 (segment (start 151.859 98.565) (end 152.959 99.665) (width 0.2) (layer "F.Cu") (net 5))
 (segment (start 154.059 100.765) (end 168.018 100.765) (width 0.2) (layer "F.Cu") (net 5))
 (segment (start 121.54 95.5675) (end 121.6575 95.685) (width 0.2) (layer "F.Cu") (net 6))
 (segment (start 135.7 95.685) (end 136.8 94.585) (width 0.2) (layer "F.Cu") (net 6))
 (segment (start 121.6575 95.685) (end 135.7 95.685) (width 0.2) (layer "F.Cu") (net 6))
 (segment (start 185.277 97.125) (end 186.377 98.225) (width 0.2) (layer "F.Cu") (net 4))
 (segment (start 121.54 93.0275) (end 121.4125 92.9) (width 0.2) (layer "F.Cu") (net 4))
 (segment (start 184.177 96.025) (end 185.277 97.125) (width 0.2) (layer "F.Cu") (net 4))
 (segment (start 200.336 98.225) (end 201.436 97.125) (width 0.2) (layer "F.Cu") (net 4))
 (segment (start 118.4 92.9) (end 117.6 93.7) (width 0.2) (layer "F.Cu") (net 4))
 (segment (start 137.9 96.025) (end 151.859 96.025) (width 0.2) (layer "F.Cu") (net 4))
 (segment (start 154.059 96.025) (end 168.018 96.025) (width 0.2) (layer "F.Cu") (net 4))
 (segment (start 170.218 96.025) (end 184.177 96.025) (width 0.2) (layer "F.Cu") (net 4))
 (segment (start 152.959 97.125) (end 154.059 96.025) (width 0.2) (layer "F.Cu") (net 4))
 (segment (start 136.8 97.125) (end 137.9 96.025) (width 0.2) (layer "F.Cu") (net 4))
 (segment (start 186.377 98.225) (end 200.336 98.225) (width 0.2) (layer "F.Cu") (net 4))
 (segment (start 216.495 96.025) (end 217.595 97.125) (width 0.2) (layer "F.Cu") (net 4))
 (segment (start 134.235 98.565) (end 135.675 97.125) (width 0.2) (layer "F.Cu") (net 4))
 (segment (start 121.4125 92.9) (end 118.4 92.9) (width 0.2) (layer "F.Cu") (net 4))
 (segment (start 118.377575 98) (end 119.7 98) (width 0.2) (layer "F.Cu") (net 4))
 (segment (start 121.54 93.0275) (end 121.6575 93.145) (width 0.2) (layer "F.Cu") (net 4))
 (segment (start 123.77 96.7) (end 125.635 98.565) (width 0.2) (layer "F.Cu") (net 4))
 (segment (start 201.436 97.125) (end 202.536 96.025) (width 0.2) (layer "F.Cu") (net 4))
 (segment (start 169.118 97.125) (end 170.218 96.025) (width 0.2) (layer "F.Cu") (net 4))
 (segment (start 125.635 98.565) (end 134.235 98.565) (width 0.2) (layer "F.Cu") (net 4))
 (segment (start 121 96.7) (end 123.77 96.7) (width 0.2) (layer "F.Cu") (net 4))
 (segment (start 151.859 96.025) (end 152.959 97.125) (width 0.2) (layer "F.Cu") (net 4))
 (segment (start 135.675 97.125) (end 136.8 97.125) (width 0.2) (layer "F.Cu") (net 4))
 (segment (start 119.7 98) (end 121 96.7) (width 0.2) (layer "F.Cu") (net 4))
 (segment (start 117.6 93.7) (end 117.6 97.222425) (width 0.2) (layer "F.Cu") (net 4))
 (segment (start 202.536 96.025) (end 216.495 96.025) (width 0.2) (layer "F.Cu") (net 4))
 (segment (start 117.6 97.222425) (end 118.377575 98) (width 0.2) (layer "F.Cu") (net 4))
 (segment (start 168.018 96.025) (end 169.118 97.125) (width 0.2) (layer "F.Cu") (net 4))
 (segment (start 135.3 90.545) (end 135.3 107.08) (width 0.2) (layer "B.Cu") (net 31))
 (segment (start 129.18 84.425) (end 135.3 90.545) (width 0.2) (layer "B.Cu") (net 31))
 (segment (start 135.3 107.08) (end 138.48 110.26) (width 0.2) (layer "B.Cu") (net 31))
 (segment (start 130.68 108.022105) (end 129.382 109.320105) (width 0.2) (layer "B.Cu") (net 29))
 (segment (start 129.382 109.320105) (end 129.382 118.942) (width 0.2) (layer "B.Cu") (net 29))
 (segment (start 130.68 88.465) (end 130.68 108.022105) (width 0.2) (layer "B.Cu") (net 29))
 (segment (start 129.382 118.942) (end 135.94 125.5) (width 0.2) (layer "B.Cu") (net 29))
 (segment (start 129.18 86.965) (end 130.68 88.465) (width 0.2) (layer "B.Cu") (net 29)))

